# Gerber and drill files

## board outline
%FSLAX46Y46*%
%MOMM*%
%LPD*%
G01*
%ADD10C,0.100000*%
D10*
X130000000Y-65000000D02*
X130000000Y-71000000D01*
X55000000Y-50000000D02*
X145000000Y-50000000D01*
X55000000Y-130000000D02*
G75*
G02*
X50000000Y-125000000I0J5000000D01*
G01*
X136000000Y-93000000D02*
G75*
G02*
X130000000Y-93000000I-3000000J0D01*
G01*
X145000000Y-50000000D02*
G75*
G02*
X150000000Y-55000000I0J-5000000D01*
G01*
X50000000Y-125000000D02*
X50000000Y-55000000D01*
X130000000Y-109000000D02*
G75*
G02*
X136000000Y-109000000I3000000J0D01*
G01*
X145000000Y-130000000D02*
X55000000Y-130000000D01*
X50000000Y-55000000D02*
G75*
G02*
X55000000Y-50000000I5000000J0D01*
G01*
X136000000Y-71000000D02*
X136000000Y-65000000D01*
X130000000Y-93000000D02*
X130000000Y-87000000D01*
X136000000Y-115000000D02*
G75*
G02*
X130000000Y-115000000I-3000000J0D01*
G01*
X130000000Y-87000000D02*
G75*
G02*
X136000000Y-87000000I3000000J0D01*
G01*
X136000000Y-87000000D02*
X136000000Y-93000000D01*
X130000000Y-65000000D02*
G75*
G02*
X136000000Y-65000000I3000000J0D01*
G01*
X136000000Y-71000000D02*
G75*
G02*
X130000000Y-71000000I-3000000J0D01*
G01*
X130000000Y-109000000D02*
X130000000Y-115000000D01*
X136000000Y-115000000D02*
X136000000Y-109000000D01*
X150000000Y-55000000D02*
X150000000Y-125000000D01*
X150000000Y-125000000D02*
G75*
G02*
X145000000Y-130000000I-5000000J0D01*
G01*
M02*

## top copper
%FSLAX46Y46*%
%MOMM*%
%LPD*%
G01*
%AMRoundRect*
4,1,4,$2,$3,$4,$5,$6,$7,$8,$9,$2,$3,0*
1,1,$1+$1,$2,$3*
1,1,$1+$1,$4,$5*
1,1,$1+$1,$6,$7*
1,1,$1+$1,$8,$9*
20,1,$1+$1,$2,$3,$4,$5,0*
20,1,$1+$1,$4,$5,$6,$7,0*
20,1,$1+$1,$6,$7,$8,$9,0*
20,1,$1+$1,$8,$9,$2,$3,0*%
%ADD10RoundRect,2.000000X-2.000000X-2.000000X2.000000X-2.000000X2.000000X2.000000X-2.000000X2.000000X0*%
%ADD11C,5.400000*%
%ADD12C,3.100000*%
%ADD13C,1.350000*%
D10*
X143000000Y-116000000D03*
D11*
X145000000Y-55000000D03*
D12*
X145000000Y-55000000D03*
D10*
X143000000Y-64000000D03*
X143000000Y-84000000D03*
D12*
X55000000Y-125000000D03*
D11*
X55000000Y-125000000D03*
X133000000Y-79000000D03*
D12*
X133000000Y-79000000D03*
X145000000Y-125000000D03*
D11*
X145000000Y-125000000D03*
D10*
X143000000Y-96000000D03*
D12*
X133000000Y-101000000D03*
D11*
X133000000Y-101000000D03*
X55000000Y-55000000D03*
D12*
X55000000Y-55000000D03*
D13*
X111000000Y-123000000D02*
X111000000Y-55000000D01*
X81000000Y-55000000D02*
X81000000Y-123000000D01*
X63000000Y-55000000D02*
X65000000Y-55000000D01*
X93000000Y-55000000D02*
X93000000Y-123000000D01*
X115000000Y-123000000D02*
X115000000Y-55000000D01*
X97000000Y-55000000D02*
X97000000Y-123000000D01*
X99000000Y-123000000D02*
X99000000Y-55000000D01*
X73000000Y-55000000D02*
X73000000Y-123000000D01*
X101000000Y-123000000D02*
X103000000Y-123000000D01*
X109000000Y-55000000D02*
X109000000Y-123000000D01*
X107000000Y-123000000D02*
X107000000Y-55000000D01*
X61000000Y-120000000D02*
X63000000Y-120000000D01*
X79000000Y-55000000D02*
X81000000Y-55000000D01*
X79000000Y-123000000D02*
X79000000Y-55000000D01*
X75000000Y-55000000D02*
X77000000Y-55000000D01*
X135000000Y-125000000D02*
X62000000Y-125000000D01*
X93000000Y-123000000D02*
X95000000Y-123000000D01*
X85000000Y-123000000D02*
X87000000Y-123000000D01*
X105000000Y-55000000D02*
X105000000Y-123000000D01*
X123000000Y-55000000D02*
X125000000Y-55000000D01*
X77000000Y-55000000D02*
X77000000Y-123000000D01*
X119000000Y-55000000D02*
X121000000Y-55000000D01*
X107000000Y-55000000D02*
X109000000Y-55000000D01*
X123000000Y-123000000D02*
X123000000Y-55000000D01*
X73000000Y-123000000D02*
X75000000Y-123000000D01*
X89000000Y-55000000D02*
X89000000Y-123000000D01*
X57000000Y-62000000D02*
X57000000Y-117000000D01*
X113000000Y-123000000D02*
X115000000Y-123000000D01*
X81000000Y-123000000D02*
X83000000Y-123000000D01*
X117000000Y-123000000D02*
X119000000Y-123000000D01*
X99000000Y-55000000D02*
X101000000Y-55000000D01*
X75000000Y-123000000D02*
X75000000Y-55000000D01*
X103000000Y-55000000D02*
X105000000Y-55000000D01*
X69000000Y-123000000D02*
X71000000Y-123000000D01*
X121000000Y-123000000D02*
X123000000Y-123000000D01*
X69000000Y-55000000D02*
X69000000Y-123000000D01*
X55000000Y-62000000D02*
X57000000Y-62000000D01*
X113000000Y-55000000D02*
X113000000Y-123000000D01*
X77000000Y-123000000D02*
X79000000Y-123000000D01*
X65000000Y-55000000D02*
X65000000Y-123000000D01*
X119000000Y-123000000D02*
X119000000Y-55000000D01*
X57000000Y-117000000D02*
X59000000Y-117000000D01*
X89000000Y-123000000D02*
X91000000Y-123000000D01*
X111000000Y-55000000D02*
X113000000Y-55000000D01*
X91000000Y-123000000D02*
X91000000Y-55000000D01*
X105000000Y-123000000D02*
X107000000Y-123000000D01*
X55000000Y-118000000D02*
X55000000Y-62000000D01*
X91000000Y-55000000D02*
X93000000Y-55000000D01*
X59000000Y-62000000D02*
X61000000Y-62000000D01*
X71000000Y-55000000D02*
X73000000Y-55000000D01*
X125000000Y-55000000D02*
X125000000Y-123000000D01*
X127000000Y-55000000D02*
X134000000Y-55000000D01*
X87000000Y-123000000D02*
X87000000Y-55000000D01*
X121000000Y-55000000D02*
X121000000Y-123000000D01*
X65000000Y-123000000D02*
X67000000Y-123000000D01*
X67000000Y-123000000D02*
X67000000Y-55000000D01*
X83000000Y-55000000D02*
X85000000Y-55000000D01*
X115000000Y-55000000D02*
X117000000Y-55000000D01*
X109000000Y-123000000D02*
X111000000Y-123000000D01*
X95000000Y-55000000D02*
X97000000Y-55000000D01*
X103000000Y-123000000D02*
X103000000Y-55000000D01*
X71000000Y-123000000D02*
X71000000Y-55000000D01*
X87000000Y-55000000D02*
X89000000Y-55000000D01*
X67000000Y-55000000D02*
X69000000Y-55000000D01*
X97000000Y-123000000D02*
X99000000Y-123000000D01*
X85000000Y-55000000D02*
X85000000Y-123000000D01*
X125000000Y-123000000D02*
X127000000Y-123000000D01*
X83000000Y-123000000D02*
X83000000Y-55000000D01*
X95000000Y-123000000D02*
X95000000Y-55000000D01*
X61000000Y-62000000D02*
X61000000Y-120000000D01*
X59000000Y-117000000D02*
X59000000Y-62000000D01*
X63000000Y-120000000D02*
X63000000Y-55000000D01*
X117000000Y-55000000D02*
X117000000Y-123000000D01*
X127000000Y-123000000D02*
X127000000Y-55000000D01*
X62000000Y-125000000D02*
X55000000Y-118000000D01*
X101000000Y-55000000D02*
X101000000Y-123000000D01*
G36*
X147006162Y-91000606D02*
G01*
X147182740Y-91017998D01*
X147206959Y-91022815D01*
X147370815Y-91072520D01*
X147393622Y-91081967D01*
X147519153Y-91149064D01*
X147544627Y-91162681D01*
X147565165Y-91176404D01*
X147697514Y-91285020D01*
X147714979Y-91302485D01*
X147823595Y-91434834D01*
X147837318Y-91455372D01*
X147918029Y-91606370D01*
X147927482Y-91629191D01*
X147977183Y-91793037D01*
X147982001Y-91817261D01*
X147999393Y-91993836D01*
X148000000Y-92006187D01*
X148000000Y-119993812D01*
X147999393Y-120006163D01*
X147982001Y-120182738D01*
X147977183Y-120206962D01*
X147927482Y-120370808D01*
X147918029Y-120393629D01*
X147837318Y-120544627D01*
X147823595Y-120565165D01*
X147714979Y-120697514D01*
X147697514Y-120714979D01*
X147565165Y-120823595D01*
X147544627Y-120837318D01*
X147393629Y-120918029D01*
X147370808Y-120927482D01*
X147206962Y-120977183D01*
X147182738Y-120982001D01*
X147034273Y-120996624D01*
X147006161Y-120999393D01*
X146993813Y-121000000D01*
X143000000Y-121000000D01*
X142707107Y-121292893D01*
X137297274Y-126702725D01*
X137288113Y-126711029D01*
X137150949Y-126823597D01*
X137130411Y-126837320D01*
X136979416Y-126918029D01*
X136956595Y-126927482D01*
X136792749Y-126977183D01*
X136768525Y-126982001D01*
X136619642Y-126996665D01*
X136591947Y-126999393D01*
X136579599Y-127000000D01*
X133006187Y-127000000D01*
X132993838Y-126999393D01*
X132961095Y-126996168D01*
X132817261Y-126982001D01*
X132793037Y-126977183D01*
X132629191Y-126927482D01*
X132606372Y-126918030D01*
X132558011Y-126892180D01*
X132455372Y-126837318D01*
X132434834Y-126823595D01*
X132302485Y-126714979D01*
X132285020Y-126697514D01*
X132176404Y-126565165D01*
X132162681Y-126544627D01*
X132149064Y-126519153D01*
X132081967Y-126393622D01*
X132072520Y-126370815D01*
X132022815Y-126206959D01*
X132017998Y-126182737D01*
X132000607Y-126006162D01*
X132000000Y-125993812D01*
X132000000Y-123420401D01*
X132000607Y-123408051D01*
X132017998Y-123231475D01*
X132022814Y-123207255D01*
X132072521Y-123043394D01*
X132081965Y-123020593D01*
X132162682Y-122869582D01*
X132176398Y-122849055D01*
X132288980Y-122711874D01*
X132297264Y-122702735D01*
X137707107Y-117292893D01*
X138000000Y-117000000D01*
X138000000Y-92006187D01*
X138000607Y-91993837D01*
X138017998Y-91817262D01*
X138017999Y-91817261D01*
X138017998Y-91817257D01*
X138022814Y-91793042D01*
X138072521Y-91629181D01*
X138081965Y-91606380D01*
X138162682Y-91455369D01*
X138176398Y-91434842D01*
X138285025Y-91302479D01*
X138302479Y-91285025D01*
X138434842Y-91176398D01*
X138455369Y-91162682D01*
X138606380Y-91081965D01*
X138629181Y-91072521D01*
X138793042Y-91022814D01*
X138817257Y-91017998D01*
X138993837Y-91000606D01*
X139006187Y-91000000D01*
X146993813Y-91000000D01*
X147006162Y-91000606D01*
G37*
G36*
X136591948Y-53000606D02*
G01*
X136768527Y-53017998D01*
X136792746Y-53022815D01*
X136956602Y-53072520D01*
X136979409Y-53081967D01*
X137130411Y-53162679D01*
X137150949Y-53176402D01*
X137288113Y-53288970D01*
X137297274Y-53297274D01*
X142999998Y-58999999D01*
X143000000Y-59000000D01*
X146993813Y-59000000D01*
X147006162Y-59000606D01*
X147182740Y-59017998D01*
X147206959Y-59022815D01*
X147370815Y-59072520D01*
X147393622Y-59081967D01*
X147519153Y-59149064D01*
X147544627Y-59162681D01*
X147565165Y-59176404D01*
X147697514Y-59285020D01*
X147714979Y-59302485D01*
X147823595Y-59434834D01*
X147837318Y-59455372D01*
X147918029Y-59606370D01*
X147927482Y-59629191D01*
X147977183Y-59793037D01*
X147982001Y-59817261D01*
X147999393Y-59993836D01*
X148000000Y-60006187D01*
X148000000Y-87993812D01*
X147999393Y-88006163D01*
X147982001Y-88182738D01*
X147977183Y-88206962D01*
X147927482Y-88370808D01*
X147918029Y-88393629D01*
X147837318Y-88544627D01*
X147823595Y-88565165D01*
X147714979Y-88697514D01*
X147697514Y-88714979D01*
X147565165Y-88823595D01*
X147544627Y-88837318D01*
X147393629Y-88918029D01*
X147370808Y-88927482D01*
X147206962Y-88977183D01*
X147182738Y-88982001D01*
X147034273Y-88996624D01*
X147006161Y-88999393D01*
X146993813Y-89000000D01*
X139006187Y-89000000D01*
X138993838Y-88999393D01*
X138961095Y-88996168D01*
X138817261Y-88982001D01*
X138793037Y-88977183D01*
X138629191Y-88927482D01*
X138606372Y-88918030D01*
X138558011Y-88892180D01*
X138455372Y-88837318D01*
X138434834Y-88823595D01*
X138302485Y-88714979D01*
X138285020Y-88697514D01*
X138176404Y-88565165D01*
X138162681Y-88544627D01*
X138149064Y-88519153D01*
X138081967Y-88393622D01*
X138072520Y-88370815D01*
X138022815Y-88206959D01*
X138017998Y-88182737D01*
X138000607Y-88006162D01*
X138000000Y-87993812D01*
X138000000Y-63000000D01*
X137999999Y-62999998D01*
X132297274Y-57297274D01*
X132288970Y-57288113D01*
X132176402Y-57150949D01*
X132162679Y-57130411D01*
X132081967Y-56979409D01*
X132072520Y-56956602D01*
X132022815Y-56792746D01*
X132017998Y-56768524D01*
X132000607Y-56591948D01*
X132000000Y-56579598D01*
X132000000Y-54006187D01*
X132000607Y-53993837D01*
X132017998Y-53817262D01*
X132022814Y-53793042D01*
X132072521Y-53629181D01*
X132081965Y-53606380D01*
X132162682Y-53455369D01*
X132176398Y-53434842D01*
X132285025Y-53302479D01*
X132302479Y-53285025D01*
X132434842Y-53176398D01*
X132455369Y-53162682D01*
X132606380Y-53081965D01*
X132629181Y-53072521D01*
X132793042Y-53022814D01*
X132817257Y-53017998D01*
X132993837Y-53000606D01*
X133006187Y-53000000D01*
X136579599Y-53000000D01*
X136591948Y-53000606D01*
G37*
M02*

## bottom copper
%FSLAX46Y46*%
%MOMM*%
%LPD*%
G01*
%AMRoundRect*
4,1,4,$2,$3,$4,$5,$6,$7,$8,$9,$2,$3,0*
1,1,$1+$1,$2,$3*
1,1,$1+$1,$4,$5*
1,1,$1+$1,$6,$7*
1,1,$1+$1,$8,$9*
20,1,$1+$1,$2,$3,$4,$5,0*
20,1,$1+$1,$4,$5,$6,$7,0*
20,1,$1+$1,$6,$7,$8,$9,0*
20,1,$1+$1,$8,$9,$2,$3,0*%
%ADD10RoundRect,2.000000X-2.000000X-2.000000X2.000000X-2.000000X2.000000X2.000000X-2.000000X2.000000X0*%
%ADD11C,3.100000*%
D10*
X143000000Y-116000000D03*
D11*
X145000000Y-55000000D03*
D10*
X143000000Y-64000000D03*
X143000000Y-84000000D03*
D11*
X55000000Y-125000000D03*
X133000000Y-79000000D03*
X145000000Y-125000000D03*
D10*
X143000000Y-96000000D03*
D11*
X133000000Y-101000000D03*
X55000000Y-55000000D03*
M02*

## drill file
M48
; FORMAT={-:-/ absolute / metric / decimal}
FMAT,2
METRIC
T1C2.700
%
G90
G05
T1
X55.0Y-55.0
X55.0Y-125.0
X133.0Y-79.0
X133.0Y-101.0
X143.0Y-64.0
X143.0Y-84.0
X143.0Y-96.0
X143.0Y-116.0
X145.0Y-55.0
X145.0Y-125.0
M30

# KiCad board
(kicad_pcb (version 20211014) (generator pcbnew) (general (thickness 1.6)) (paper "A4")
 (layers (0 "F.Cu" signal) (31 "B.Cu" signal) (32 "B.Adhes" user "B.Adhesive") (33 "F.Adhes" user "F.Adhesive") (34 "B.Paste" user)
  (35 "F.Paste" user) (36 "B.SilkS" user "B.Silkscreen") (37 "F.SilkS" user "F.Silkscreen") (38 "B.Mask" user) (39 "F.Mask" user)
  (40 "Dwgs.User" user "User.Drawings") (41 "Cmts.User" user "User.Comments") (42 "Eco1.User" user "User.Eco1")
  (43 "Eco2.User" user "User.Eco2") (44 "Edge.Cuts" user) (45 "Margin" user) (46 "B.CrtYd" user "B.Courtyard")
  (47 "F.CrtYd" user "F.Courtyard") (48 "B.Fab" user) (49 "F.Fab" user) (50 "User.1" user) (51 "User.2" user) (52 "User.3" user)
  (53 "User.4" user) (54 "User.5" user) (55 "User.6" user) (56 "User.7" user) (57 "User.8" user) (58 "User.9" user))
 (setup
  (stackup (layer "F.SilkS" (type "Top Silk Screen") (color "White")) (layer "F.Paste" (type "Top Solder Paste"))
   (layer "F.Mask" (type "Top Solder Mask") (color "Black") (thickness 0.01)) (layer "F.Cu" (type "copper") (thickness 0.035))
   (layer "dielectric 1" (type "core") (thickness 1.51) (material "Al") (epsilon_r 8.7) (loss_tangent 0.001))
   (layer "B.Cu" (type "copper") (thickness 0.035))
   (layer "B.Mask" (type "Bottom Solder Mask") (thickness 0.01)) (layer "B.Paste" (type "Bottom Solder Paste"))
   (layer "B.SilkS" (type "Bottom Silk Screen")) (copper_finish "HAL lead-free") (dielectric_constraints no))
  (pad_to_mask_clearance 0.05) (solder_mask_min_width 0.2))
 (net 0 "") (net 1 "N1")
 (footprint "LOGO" (layer "F.Cu") (at 118 113)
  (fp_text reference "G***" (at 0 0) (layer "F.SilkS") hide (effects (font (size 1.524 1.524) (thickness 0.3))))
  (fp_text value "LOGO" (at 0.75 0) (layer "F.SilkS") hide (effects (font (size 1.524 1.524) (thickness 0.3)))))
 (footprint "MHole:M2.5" (layer "F.Cu") (at 143 116)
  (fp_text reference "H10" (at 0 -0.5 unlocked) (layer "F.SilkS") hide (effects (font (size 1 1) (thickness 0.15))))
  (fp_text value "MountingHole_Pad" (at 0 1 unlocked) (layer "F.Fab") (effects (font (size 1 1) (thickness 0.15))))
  (pad "1" thru_hole roundrect (at 0 0) (size 8 8) (drill 2.7) (layers *.Cu *.Mask) (roundrect_rratio 0.25) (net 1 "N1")))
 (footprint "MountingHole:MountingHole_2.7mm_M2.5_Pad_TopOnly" (layer "F.Cu") (at 145 55)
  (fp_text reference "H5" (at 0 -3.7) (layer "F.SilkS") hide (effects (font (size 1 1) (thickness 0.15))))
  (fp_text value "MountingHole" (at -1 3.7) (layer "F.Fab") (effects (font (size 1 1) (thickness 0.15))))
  (pad "1" connect circle (at 0 0) (size 5.4 5.4) (layers "F.Cu" "F.Mask"))
  (pad "1" thru_hole circle (at 0 0) (size 3.1 3.1) (drill 2.7) (layers *.Cu *.Mask)))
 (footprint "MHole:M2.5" (layer "F.Cu") (at 143 64)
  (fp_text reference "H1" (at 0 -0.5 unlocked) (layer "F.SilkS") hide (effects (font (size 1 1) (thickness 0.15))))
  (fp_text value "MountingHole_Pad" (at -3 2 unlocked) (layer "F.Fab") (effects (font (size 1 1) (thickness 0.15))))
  (pad "1" thru_hole roundrect (at 0 0) (size 8 8) (drill 2.7) (layers *.Cu *.Mask) (roundrect_rratio 0.25) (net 1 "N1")))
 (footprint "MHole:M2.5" (layer "F.Cu") (at 143 84)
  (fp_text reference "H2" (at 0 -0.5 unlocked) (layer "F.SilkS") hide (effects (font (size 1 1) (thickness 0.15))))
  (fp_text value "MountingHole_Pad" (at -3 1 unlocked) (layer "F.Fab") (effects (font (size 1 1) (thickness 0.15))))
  (pad "1" thru_hole roundrect (at 0 0) (size 8 8) (drill 2.7) (layers *.Cu *.Mask) (roundrect_rratio 0.25) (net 1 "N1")))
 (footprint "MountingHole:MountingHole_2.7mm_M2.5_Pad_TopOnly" (layer "F.Cu") (at 55 125)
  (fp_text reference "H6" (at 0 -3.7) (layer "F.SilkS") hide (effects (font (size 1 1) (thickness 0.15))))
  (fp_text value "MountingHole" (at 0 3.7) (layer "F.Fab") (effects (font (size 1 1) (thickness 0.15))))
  (pad "1" thru_hole circle (at 0 0) (size 3.1 3.1) (drill 2.7) (layers *.Cu *.Mask))
  (pad "1" connect circle (at 0 0) (size 5.4 5.4) (layers "F.Cu" "F.Mask")))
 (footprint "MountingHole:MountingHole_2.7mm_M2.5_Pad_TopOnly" (layer "F.Cu") (at 133 79)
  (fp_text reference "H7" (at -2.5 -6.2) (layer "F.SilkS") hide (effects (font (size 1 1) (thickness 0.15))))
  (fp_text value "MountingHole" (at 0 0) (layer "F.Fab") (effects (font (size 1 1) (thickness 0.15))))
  (pad "1" connect circle (at 0 0) (size 5.4 5.4) (layers "F.Cu" "F.Mask"))
  (pad "1" thru_hole circle (at 0 0) (size 3.1 3.1) (drill 2.7) (layers *.Cu *.Mask)))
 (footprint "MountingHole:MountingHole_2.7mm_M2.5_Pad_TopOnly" (layer "F.Cu") (at 145 125)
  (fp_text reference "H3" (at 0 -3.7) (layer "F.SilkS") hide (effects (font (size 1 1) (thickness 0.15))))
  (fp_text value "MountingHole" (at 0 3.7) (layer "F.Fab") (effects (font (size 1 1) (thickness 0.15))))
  (pad "1" thru_hole circle (at 0 0) (size 3.1 3.1) (drill 2.7) (layers *.Cu *.Mask))
  (pad "1" connect circle (at 0 0) (size 5.4 5.4) (layers "F.Cu" "F.Mask")))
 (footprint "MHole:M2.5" (layer "F.Cu") (at 143 96)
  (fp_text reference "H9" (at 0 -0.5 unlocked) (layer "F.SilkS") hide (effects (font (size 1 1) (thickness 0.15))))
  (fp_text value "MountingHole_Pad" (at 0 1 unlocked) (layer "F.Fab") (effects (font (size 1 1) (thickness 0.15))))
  (pad "1" thru_hole roundrect (at 0 0) (size 8 8) (drill 2.7) (layers *.Cu *.Mask) (roundrect_rratio 0.25) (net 1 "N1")))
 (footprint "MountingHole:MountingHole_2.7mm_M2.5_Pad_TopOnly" (layer "F.Cu") (at 133 101)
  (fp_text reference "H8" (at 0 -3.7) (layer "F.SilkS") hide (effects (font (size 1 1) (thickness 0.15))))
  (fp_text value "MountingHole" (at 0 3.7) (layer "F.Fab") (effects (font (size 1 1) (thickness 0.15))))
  (pad "1" thru_hole circle (at 0 0) (size 3.1 3.1) (drill 2.7) (layers *.Cu *.Mask))
  (pad "1" connect circle (at 0 0) (size 5.4 5.4) (layers "F.Cu" "F.Mask")))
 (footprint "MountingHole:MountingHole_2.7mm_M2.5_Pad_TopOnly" (layer "F.Cu") (at 55 55)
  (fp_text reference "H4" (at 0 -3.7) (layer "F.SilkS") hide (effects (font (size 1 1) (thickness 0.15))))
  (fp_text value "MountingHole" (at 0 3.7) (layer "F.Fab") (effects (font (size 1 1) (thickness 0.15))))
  (pad "1" connect circle (at 0 0) (size 5.4 5.4) (layers "F.Cu" "F.Mask"))
  (pad "1" thru_hole circle (at 0 0) (size 3.1 3.1) (drill 2.7) (layers *.Cu *.Mask)))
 (gr_line (start 130 65) (end 130 71) (layer "Edge.Cuts") (width 0.1))
 (gr_line (start 55 50) (end 145 50) (layer "Edge.Cuts") (width 0.1))
 (gr_arc (start 55 130) (mid 51.464466 128.535534) (end 50 125) (layer "Edge.Cuts") (width 0.1))
 (gr_arc (start 136 93) (mid 133 96) (end 130 93) (layer "Edge.Cuts") (width 0.1))
 (gr_arc (start 145 50) (mid 148.535534 51.464466) (end 150 55) (layer "Edge.Cuts") (width 0.1))
 (gr_line (start 50 125) (end 50 55) (layer "Edge.Cuts") (width 0.1))
 (gr_arc (start 130 109) (mid 133 106) (end 136 109) (layer "Edge.Cuts") (width 0.1))
 (gr_line (start 145 130) (end 55 130) (layer "Edge.Cuts") (width 0.1))
 (gr_arc (start 50 55) (mid 51.464466 51.464466) (end 55 50) (layer "Edge.Cuts") (width 0.1))
 (gr_line (start 136 71) (end 136 65) (layer "Edge.Cuts") (width 0.1))
 (gr_line (start 130 93) (end 130 87) (layer "Edge.Cuts") (width 0.1))
 (gr_arc (start 136 115) (mid 133 118) (end 130 115) (layer "Edge.Cuts") (width 0.1))
 (gr_arc (start 130 87) (mid 133 84) (end 136 87) (layer "Edge.Cuts") (width 0.1))
 (gr_line (start 136 87) (end 136 93) (layer "Edge.Cuts") (width 0.1))
 (gr_arc (start 130 65) (mid 133 62) (end 136 65) (layer "Edge.Cuts") (width 0.1))
 (gr_arc (start 136 71) (mid 133 74) (end 130 71) (layer "Edge.Cuts") (width 0.1))
 (gr_line (start 130 109) (end 130 115) (layer "Edge.Cuts") (width 0.1))
 (gr_line (start 136 115) (end 136 109) (layer "Edge.Cuts") (width 0.1))
 (gr_line (start 150 55) (end 150 125) (layer "Edge.Cuts") (width 0.1))
 (gr_arc (start 150 125) (mid 148.535534 128.535534) (end 145 130) (layer "Edge.Cuts") (width 0.1))
 (segment (start 111 123) (end 111 55) (width 1.35) (layer "F.Cu") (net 1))
 (segment (start 81 55) (end 81 123) (width 1.35) (layer "F.Cu") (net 1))
 (segment (start 63 55) (end 65 55) (width 1.35) (layer "F.Cu") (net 1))
 (segment (start 93 55) (end 93 123) (width 1.35) (layer "F.Cu") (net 1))
 (segment (start 115 123) (end 115 55) (width 1.35) (layer "F.Cu") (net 1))
 (segment (start 97 55) (end 97 123) (width 1.35) (layer "F.Cu") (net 1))
 (segment (start 99 123) (end 99 55) (width 1.35) (layer "F.Cu") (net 1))
 (segment (start 73 55) (end 73 123) (width 1.35) (layer "F.Cu") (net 1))
 (segment (start 101 123) (end 103 123) (width 1.35) (layer "F.Cu") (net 1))
 (segment (start 109 55) (end 109 123) (width 1.35) (layer "F.Cu") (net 1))
 (segment (start 107 123) (end 107 55) (width 1.35) (layer "F.Cu") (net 1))
 (segment (start 61 120) (end 63 120) (width 1.35) (layer "F.Cu") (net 1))
 (segment (start 79 55) (end 81 55) (width 1.35) (layer "F.Cu") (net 1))
 (segment (start 79 123) (end 79 55) (width 1.35) (layer "F.Cu") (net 1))
 (segment (start 75 55) (end 77 55) (width 1.35) (layer "F.Cu") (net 1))
 (segment (start 135 125) (end 62 125) (width 1.35) (layer "F.Cu") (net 1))
 (segment (start 93 123) (end 95 123) (width 1.35) (layer "F.Cu") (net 1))
 (segment (start 85 123) (end 87 123) (width 1.35) (layer "F.Cu") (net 1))
 (segment (start 105 55) (end 105 123) (width 1.35) (layer "F.Cu") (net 1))
 (segment (start 123 55) (end 125 55) (width 1.35) (layer "F.Cu") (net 1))
 (segment (start 77 55) (end 77 123) (width 1.35) (layer "F.Cu") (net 1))
 (segment (start 119 55) (end 121 55) (width 1.35) (layer "F.Cu") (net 1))
 (segment (start 107 55) (end 109 55) (width 1.35) (layer "F.Cu") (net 1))
 (segment (start 123 123) (end 123 55) (width 1.35) (layer "F.Cu") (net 1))
 (segment (start 73 123) (end 75 123) (width 1.35) (layer "F.Cu") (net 1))
 (segment (start 89 55) (end 89 123) (width 1.35) (layer "F.Cu") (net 1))
 (segment (start 57 62) (end 57 117) (width 1.35) (layer "F.Cu") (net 1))
 (segment (start 113 123) (end 115 123) (width 1.35) (layer "F.Cu") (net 1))
 (segment (start 81 123) (end 83 123) (width 1.35) (layer "F.Cu") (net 1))
 (segment (start 117 123) (end 119 123) (width 1.35) (layer "F.Cu") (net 1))
 (segment (start 99 55) (end 101 55) (width 1.35) (layer "F.Cu") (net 1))
 (segment (start 75 123) (end 75 55) (width 1.35) (layer "F.Cu") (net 1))
 (segment (start 103 55) (end 105 55) (width 1.35) (layer "F.Cu") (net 1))
 (segment (start 69 123) (end 71 123) (width 1.35) (layer "F.Cu") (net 1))
 (segment (start 121 123) (end 123 123) (width 1.35) (layer "F.Cu") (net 1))
 (segment (start 69 55) (end 69 123) (width 1.35) (layer "F.Cu") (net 1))
 (segment (start 55 62) (end 57 62) (width 1.35) (layer "F.Cu") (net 1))
 (segment (start 113 55) (end 113 123) (width 1.35) (layer "F.Cu") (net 1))
 (segment (start 77 123) (end 79 123) (width 1.35) (layer "F.Cu") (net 1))
 (segment (start 65 55) (end 65 123) (width 1.35) (layer "F.Cu") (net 1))
 (segment (start 119 123) (end 119 55) (width 1.35) (layer "F.Cu") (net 1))
 (segment (start 57 117) (end 59 117) (width 1.35) (layer "F.Cu") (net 1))
 (segment (start 89 123) (end 91 123) (width 1.35) (layer "F.Cu") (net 1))
 (segment (start 111 55) (end 113 55) (width 1.35) (layer "F.Cu") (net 1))
 (segment (start 91 123) (end 91 55) (width 1.35) (layer "F.Cu") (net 1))
 (segment (start 105 123) (end 107 123) (width 1.35) (layer "F.Cu") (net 1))
 (segment (start 55 118) (end 55 62) (width 1.35) (layer "F.Cu") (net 1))
 (segment (start 91 55) (end 93 55) (width 1.35) (layer "F.Cu") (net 1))
 (segment (start 59 62) (end 61 62) (width 1.35) (layer "F.Cu") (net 1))
 (segment (start 71 55) (end 73 55) (width 1.35) (layer "F.Cu") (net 1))
 (segment (start 125 55) (end 125 123) (width 1.35) (layer "F.Cu") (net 1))
 (segment (start 127 55) (end 134 55) (width 1.35) (layer "F.Cu") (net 1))
 (segment (start 87 123) (end 87 55) (width 1.35) (layer "F.Cu") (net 1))
 (segment (start 121 55) (end 121 123) (width 1.35) (layer "F.Cu") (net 1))
 (segment (start 65 123) (end 67 123) (width 1.35) (layer "F.Cu") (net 1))
 (segment (start 67 123) (end 67 55) (width 1.35) (layer "F.Cu") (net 1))
 (segment (start 83 55) (end 85 55) (width 1.35) (layer "F.Cu") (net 1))
 (segment (start 115 55) (end 117 55) (width 1.35) (layer "F.Cu") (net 1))
 (segment (start 109 123) (end 111 123) (width 1.35) (layer "F.Cu") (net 1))
 (segment (start 95 55) (end 97 55) (width 1.35) (layer "F.Cu") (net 1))
 (segment (start 103 123) (end 103 55) (width 1.35) (layer "F.Cu") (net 1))
 (segment (start 71 123) (end 71 55) (width 1.35) (layer "F.Cu") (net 1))
 (segment (start 87 55) (end 89 55) (width 1.35) (layer "F.Cu") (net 1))
 (segment (start 67 55) (end 69 55) (width 1.35) (layer "F.Cu") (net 1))
 (segment (start 97 123) (end 99 123) (width 1.35) (layer "F.Cu") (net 1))
 (segment (start 85 55) (end 85 123) (width 1.35) (layer "F.Cu") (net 1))
 (segment (start 125 123) (end 127 123) (width 1.35) (layer "F.Cu") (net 1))
 (segment (start 83 123) (end 83 55) (width 1.35) (layer "F.Cu") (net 1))
 (segment (start 95 123) (end 95 55) (width 1.35) (layer "F.Cu") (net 1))
 (segment (start 61 62) (end 61 120) (width 1.35) (layer "F.Cu") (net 1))
 (segment (start 59 117) (end 59 62) (width 1.35) (layer "F.Cu") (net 1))
 (segment (start 63 120) (end 63 55) (width 1.35) (layer "F.Cu") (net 1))
 (segment (start 117 55) (end 117 123) (width 1.35) (layer "F.Cu") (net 1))
 (segment (start 127 123) (end 127 55) (width 1.35) (layer "F.Cu") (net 1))
 (segment (start 62 125) (end 55 118) (width 1.35) (layer "F.Cu") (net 1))
 (segment (start 101 55) (end 101 123) (width 1.35) (layer "F.Cu") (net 1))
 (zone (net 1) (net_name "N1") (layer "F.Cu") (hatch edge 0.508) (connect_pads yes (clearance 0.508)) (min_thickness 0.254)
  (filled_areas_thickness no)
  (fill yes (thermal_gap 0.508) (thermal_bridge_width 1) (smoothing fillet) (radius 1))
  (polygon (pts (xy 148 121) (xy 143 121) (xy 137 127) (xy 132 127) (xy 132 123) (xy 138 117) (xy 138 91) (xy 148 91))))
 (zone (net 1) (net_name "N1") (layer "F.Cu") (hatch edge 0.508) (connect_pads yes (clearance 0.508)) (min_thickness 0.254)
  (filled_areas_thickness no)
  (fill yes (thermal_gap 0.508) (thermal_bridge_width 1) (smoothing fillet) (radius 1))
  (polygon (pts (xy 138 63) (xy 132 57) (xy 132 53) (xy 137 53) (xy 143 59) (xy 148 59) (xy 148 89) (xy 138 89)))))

